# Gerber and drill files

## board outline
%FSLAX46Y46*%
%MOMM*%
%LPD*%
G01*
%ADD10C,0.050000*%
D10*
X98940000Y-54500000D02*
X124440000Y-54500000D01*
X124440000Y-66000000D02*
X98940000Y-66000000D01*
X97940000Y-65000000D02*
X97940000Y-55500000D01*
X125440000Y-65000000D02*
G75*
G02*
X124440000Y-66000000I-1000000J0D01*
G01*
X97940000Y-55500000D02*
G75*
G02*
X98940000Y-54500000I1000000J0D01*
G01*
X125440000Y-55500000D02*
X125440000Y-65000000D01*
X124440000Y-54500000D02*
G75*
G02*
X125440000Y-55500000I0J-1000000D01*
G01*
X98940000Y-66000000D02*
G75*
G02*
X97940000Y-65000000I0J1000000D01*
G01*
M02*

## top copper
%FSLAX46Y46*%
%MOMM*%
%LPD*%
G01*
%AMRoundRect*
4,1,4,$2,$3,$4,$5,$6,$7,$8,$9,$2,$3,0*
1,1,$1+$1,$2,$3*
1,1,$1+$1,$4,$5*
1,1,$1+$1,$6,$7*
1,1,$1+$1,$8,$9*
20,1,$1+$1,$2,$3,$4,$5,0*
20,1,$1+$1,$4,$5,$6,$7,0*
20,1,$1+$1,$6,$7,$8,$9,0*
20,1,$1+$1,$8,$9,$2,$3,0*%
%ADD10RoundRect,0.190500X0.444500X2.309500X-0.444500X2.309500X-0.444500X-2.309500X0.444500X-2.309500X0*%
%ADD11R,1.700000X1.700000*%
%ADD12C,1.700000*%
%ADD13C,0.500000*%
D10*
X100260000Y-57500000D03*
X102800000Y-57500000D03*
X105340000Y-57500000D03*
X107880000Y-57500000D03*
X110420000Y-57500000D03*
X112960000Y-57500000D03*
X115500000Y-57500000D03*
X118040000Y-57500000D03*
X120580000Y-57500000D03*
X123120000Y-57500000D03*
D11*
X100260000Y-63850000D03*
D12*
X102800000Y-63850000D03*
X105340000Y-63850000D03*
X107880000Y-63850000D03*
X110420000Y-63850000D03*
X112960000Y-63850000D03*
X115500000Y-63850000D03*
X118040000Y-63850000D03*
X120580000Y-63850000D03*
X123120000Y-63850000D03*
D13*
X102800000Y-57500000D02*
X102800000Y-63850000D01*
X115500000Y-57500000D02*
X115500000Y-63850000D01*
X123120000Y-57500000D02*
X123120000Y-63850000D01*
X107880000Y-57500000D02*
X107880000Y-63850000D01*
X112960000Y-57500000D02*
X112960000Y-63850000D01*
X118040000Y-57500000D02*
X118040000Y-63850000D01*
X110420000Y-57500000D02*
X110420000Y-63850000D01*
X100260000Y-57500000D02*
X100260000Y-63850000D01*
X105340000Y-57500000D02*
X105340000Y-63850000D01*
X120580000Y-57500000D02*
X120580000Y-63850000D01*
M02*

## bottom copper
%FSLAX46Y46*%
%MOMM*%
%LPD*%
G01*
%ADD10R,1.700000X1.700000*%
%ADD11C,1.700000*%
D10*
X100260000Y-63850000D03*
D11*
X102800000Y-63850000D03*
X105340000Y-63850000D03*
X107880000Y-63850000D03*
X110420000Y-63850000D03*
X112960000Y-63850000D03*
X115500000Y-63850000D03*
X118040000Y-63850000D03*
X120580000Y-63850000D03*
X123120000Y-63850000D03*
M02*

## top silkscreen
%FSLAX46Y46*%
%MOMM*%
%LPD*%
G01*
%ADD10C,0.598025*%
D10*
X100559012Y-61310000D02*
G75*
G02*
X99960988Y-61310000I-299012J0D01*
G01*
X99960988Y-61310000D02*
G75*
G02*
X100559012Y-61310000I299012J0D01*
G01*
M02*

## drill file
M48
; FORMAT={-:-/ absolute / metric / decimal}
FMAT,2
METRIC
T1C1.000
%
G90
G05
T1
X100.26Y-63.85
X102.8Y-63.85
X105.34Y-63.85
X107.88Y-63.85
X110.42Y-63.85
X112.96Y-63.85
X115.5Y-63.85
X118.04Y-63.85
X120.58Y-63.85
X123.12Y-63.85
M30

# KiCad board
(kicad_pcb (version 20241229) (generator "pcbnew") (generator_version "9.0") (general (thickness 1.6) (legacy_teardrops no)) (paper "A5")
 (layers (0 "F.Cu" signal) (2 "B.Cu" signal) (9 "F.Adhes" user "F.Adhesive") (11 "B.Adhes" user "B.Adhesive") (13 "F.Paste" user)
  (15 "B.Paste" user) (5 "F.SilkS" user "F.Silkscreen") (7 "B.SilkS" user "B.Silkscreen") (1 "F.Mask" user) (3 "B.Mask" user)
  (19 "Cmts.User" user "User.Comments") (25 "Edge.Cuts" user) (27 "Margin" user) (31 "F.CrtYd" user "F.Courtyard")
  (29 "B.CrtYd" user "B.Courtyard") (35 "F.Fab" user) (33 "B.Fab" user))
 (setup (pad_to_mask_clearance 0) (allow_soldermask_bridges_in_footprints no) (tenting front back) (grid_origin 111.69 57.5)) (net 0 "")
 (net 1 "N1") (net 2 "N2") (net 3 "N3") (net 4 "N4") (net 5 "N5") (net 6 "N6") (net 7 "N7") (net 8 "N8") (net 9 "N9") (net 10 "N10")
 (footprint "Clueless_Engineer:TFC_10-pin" (layer "F.Cu") (at 111.69 57.5)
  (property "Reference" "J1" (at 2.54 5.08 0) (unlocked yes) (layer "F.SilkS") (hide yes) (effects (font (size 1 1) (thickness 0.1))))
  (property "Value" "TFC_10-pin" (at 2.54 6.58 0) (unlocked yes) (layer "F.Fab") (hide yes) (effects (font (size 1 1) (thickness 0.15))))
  (pad "1" connect roundrect (at -11.43 0 180) (size 1.27 5) (layers "F.Cu" "F.Mask") (roundrect_rratio 0.15) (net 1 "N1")
   (thermal_bridge_angle 45))
  (pad "2" connect roundrect (at -8.89 0 180) (size 1.27 5) (layers "F.Cu" "F.Mask") (roundrect_rratio 0.15) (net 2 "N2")
   (thermal_bridge_angle 45))
  (pad "3" connect roundrect (at -6.35 0 180) (size 1.27 5) (layers "F.Cu" "F.Mask") (roundrect_rratio 0.15) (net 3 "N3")
   (thermal_bridge_angle 45))
  (pad "4" connect roundrect (at -3.81 0 180) (size 1.27 5) (layers "F.Cu" "F.Mask") (roundrect_rratio 0.15) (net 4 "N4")
   (thermal_bridge_angle 45))
  (pad "5" connect roundrect (at -1.27 0 180) (size 1.27 5) (layers "F.Cu" "F.Mask") (roundrect_rratio 0.15) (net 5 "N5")
   (thermal_bridge_angle 45))
  (pad "6" connect roundrect (at 1.27 0 180) (size 1.27 5) (layers "F.Cu" "F.Mask") (roundrect_rratio 0.15) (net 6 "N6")
   (thermal_bridge_angle 45))
  (pad "7" connect roundrect (at 3.81 0 180) (size 1.27 5) (layers "F.Cu" "F.Mask") (roundrect_rratio 0.15) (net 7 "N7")
   (thermal_bridge_angle 45))
  (pad "8" connect roundrect (at 6.35 0 180) (size 1.27 5) (layers "F.Cu" "F.Mask") (roundrect_rratio 0.15) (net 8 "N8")
   (thermal_bridge_angle 45))
  (pad "9" connect roundrect (at 8.89 0 180) (size 1.27 5) (layers "F.Cu" "F.Mask") (roundrect_rratio 0.15) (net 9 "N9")
   (thermal_bridge_angle 45))
  (pad "10" connect roundrect (at 11.43 0 180) (size 1.27 5) (layers "F.Cu" "F.Mask") (roundrect_rratio 0.15) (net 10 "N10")
   (thermal_bridge_angle 45)))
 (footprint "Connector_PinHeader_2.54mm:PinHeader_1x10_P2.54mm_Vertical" (layer "B.Cu") (at 100.26 63.85 -90)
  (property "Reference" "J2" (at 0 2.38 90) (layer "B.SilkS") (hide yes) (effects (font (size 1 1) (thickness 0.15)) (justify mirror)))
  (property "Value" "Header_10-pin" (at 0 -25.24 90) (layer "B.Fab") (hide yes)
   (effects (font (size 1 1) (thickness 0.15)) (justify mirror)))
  (pad "1" thru_hole rect (at 0 0 270) (size 1.7 1.7) (drill 1) (layers "*.Cu" "*.Mask") (remove_unused_layers no) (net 1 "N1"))
  (pad "2" thru_hole circle (at 0 -2.54 270) (size 1.7 1.7) (drill 1) (layers "*.Cu" "*.Mask") (remove_unused_layers no) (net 2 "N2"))
  (pad "3" thru_hole circle (at 0 -5.08 270) (size 1.7 1.7) (drill 1) (layers "*.Cu" "*.Mask") (remove_unused_layers no) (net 3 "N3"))
  (pad "4" thru_hole circle (at 0 -7.62 270) (size 1.7 1.7) (drill 1) (layers "*.Cu" "*.Mask") (remove_unused_layers no) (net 4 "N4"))
  (pad "5" thru_hole circle (at 0 -10.16 270) (size 1.7 1.7) (drill 1) (layers "*.Cu" "*.Mask") (remove_unused_layers no) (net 5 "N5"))
  (pad "6" thru_hole circle (at 0 -12.7 270) (size 1.7 1.7) (drill 1) (layers "*.Cu" "*.Mask") (remove_unused_layers no) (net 6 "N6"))
  (pad "7" thru_hole circle (at 0 -15.24 270) (size 1.7 1.7) (drill 1) (layers "*.Cu" "*.Mask") (remove_unused_layers no) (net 7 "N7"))
  (pad "8" thru_hole circle (at 0 -17.78 270) (size 1.7 1.7) (drill 1) (layers "*.Cu" "*.Mask") (remove_unused_layers no) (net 8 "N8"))
  (pad "9" thru_hole circle (at 0 -20.32 270) (size 1.7 1.7) (drill 1) (layers "*.Cu" "*.Mask") (remove_unused_layers no) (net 9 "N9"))
  (pad "10" thru_hole circle (at 0 -22.86 270) (size 1.7 1.7) (drill 1) (layers "*.Cu" "*.Mask") (remove_unused_layers no) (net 10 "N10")))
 (gr_circle (center 100.26 61.31) (end 100.791817 61.442295) (stroke (width 0.1) (type solid)) (fill yes) (layer "F.SilkS"))
 (gr_line (start 98.94 54.5) (end 124.44 54.5) (stroke (width 0.05) (type default)) (layer "Edge.Cuts"))
 (gr_line (start 124.44 66) (end 98.94 66) (stroke (width 0.05) (type default)) (layer "Edge.Cuts"))
 (gr_line (start 97.94 65) (end 97.94 55.5) (stroke (width 0.05) (type default)) (layer "Edge.Cuts"))
 (gr_arc (start 125.44 65) (mid 125.147107 65.707107) (end 124.44 66) (stroke (width 0.05) (type default)) (layer "Edge.Cuts"))
 (gr_arc (start 97.94 55.5) (mid 98.232893 54.792893) (end 98.94 54.5) (stroke (width 0.05) (type default)) (layer "Edge.Cuts"))
 (gr_line (start 125.44 55.5) (end 125.44 65) (stroke (width 0.05) (type default)) (layer "Edge.Cuts"))
 (gr_arc (start 124.44 54.5) (mid 125.147107 54.792893) (end 125.44 55.5) (stroke (width 0.05) (type default)) (layer "Edge.Cuts"))
 (gr_arc (start 98.94 66) (mid 98.232893 65.707107) (end 97.94 65) (stroke (width 0.05) (type default)) (layer "Edge.Cuts"))
 (segment (start 102.8 57.5) (end 102.8 63.85) (width 0.5) (layer "F.Cu") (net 2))
 (segment (start 115.5 57.5) (end 115.5 63.85) (width 0.5) (layer "F.Cu") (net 7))
 (segment (start 123.12 57.5) (end 123.12 63.85) (width 0.5) (layer "F.Cu") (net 10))
 (segment (start 107.88 57.5) (end 107.88 63.85) (width 0.5) (layer "F.Cu") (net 4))
 (segment (start 112.96 57.5) (end 112.96 63.85) (width 0.5) (layer "F.Cu") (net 6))
 (segment (start 118.04 57.5) (end 118.04 63.85) (width 0.5) (layer "F.Cu") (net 8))
 (segment (start 110.42 57.5) (end 110.42 63.85) (width 0.5) (layer "F.Cu") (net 5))
 (segment (start 100.26 57.5) (end 100.26 63.85) (width 0.5) (layer "F.Cu") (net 1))
 (segment (start 105.34 57.5) (end 105.34 63.85) (width 0.5) (layer "F.Cu") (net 3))
 (segment (start 120.58 57.5) (end 120.58 63.85) (width 0.5) (layer "F.Cu") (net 9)))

